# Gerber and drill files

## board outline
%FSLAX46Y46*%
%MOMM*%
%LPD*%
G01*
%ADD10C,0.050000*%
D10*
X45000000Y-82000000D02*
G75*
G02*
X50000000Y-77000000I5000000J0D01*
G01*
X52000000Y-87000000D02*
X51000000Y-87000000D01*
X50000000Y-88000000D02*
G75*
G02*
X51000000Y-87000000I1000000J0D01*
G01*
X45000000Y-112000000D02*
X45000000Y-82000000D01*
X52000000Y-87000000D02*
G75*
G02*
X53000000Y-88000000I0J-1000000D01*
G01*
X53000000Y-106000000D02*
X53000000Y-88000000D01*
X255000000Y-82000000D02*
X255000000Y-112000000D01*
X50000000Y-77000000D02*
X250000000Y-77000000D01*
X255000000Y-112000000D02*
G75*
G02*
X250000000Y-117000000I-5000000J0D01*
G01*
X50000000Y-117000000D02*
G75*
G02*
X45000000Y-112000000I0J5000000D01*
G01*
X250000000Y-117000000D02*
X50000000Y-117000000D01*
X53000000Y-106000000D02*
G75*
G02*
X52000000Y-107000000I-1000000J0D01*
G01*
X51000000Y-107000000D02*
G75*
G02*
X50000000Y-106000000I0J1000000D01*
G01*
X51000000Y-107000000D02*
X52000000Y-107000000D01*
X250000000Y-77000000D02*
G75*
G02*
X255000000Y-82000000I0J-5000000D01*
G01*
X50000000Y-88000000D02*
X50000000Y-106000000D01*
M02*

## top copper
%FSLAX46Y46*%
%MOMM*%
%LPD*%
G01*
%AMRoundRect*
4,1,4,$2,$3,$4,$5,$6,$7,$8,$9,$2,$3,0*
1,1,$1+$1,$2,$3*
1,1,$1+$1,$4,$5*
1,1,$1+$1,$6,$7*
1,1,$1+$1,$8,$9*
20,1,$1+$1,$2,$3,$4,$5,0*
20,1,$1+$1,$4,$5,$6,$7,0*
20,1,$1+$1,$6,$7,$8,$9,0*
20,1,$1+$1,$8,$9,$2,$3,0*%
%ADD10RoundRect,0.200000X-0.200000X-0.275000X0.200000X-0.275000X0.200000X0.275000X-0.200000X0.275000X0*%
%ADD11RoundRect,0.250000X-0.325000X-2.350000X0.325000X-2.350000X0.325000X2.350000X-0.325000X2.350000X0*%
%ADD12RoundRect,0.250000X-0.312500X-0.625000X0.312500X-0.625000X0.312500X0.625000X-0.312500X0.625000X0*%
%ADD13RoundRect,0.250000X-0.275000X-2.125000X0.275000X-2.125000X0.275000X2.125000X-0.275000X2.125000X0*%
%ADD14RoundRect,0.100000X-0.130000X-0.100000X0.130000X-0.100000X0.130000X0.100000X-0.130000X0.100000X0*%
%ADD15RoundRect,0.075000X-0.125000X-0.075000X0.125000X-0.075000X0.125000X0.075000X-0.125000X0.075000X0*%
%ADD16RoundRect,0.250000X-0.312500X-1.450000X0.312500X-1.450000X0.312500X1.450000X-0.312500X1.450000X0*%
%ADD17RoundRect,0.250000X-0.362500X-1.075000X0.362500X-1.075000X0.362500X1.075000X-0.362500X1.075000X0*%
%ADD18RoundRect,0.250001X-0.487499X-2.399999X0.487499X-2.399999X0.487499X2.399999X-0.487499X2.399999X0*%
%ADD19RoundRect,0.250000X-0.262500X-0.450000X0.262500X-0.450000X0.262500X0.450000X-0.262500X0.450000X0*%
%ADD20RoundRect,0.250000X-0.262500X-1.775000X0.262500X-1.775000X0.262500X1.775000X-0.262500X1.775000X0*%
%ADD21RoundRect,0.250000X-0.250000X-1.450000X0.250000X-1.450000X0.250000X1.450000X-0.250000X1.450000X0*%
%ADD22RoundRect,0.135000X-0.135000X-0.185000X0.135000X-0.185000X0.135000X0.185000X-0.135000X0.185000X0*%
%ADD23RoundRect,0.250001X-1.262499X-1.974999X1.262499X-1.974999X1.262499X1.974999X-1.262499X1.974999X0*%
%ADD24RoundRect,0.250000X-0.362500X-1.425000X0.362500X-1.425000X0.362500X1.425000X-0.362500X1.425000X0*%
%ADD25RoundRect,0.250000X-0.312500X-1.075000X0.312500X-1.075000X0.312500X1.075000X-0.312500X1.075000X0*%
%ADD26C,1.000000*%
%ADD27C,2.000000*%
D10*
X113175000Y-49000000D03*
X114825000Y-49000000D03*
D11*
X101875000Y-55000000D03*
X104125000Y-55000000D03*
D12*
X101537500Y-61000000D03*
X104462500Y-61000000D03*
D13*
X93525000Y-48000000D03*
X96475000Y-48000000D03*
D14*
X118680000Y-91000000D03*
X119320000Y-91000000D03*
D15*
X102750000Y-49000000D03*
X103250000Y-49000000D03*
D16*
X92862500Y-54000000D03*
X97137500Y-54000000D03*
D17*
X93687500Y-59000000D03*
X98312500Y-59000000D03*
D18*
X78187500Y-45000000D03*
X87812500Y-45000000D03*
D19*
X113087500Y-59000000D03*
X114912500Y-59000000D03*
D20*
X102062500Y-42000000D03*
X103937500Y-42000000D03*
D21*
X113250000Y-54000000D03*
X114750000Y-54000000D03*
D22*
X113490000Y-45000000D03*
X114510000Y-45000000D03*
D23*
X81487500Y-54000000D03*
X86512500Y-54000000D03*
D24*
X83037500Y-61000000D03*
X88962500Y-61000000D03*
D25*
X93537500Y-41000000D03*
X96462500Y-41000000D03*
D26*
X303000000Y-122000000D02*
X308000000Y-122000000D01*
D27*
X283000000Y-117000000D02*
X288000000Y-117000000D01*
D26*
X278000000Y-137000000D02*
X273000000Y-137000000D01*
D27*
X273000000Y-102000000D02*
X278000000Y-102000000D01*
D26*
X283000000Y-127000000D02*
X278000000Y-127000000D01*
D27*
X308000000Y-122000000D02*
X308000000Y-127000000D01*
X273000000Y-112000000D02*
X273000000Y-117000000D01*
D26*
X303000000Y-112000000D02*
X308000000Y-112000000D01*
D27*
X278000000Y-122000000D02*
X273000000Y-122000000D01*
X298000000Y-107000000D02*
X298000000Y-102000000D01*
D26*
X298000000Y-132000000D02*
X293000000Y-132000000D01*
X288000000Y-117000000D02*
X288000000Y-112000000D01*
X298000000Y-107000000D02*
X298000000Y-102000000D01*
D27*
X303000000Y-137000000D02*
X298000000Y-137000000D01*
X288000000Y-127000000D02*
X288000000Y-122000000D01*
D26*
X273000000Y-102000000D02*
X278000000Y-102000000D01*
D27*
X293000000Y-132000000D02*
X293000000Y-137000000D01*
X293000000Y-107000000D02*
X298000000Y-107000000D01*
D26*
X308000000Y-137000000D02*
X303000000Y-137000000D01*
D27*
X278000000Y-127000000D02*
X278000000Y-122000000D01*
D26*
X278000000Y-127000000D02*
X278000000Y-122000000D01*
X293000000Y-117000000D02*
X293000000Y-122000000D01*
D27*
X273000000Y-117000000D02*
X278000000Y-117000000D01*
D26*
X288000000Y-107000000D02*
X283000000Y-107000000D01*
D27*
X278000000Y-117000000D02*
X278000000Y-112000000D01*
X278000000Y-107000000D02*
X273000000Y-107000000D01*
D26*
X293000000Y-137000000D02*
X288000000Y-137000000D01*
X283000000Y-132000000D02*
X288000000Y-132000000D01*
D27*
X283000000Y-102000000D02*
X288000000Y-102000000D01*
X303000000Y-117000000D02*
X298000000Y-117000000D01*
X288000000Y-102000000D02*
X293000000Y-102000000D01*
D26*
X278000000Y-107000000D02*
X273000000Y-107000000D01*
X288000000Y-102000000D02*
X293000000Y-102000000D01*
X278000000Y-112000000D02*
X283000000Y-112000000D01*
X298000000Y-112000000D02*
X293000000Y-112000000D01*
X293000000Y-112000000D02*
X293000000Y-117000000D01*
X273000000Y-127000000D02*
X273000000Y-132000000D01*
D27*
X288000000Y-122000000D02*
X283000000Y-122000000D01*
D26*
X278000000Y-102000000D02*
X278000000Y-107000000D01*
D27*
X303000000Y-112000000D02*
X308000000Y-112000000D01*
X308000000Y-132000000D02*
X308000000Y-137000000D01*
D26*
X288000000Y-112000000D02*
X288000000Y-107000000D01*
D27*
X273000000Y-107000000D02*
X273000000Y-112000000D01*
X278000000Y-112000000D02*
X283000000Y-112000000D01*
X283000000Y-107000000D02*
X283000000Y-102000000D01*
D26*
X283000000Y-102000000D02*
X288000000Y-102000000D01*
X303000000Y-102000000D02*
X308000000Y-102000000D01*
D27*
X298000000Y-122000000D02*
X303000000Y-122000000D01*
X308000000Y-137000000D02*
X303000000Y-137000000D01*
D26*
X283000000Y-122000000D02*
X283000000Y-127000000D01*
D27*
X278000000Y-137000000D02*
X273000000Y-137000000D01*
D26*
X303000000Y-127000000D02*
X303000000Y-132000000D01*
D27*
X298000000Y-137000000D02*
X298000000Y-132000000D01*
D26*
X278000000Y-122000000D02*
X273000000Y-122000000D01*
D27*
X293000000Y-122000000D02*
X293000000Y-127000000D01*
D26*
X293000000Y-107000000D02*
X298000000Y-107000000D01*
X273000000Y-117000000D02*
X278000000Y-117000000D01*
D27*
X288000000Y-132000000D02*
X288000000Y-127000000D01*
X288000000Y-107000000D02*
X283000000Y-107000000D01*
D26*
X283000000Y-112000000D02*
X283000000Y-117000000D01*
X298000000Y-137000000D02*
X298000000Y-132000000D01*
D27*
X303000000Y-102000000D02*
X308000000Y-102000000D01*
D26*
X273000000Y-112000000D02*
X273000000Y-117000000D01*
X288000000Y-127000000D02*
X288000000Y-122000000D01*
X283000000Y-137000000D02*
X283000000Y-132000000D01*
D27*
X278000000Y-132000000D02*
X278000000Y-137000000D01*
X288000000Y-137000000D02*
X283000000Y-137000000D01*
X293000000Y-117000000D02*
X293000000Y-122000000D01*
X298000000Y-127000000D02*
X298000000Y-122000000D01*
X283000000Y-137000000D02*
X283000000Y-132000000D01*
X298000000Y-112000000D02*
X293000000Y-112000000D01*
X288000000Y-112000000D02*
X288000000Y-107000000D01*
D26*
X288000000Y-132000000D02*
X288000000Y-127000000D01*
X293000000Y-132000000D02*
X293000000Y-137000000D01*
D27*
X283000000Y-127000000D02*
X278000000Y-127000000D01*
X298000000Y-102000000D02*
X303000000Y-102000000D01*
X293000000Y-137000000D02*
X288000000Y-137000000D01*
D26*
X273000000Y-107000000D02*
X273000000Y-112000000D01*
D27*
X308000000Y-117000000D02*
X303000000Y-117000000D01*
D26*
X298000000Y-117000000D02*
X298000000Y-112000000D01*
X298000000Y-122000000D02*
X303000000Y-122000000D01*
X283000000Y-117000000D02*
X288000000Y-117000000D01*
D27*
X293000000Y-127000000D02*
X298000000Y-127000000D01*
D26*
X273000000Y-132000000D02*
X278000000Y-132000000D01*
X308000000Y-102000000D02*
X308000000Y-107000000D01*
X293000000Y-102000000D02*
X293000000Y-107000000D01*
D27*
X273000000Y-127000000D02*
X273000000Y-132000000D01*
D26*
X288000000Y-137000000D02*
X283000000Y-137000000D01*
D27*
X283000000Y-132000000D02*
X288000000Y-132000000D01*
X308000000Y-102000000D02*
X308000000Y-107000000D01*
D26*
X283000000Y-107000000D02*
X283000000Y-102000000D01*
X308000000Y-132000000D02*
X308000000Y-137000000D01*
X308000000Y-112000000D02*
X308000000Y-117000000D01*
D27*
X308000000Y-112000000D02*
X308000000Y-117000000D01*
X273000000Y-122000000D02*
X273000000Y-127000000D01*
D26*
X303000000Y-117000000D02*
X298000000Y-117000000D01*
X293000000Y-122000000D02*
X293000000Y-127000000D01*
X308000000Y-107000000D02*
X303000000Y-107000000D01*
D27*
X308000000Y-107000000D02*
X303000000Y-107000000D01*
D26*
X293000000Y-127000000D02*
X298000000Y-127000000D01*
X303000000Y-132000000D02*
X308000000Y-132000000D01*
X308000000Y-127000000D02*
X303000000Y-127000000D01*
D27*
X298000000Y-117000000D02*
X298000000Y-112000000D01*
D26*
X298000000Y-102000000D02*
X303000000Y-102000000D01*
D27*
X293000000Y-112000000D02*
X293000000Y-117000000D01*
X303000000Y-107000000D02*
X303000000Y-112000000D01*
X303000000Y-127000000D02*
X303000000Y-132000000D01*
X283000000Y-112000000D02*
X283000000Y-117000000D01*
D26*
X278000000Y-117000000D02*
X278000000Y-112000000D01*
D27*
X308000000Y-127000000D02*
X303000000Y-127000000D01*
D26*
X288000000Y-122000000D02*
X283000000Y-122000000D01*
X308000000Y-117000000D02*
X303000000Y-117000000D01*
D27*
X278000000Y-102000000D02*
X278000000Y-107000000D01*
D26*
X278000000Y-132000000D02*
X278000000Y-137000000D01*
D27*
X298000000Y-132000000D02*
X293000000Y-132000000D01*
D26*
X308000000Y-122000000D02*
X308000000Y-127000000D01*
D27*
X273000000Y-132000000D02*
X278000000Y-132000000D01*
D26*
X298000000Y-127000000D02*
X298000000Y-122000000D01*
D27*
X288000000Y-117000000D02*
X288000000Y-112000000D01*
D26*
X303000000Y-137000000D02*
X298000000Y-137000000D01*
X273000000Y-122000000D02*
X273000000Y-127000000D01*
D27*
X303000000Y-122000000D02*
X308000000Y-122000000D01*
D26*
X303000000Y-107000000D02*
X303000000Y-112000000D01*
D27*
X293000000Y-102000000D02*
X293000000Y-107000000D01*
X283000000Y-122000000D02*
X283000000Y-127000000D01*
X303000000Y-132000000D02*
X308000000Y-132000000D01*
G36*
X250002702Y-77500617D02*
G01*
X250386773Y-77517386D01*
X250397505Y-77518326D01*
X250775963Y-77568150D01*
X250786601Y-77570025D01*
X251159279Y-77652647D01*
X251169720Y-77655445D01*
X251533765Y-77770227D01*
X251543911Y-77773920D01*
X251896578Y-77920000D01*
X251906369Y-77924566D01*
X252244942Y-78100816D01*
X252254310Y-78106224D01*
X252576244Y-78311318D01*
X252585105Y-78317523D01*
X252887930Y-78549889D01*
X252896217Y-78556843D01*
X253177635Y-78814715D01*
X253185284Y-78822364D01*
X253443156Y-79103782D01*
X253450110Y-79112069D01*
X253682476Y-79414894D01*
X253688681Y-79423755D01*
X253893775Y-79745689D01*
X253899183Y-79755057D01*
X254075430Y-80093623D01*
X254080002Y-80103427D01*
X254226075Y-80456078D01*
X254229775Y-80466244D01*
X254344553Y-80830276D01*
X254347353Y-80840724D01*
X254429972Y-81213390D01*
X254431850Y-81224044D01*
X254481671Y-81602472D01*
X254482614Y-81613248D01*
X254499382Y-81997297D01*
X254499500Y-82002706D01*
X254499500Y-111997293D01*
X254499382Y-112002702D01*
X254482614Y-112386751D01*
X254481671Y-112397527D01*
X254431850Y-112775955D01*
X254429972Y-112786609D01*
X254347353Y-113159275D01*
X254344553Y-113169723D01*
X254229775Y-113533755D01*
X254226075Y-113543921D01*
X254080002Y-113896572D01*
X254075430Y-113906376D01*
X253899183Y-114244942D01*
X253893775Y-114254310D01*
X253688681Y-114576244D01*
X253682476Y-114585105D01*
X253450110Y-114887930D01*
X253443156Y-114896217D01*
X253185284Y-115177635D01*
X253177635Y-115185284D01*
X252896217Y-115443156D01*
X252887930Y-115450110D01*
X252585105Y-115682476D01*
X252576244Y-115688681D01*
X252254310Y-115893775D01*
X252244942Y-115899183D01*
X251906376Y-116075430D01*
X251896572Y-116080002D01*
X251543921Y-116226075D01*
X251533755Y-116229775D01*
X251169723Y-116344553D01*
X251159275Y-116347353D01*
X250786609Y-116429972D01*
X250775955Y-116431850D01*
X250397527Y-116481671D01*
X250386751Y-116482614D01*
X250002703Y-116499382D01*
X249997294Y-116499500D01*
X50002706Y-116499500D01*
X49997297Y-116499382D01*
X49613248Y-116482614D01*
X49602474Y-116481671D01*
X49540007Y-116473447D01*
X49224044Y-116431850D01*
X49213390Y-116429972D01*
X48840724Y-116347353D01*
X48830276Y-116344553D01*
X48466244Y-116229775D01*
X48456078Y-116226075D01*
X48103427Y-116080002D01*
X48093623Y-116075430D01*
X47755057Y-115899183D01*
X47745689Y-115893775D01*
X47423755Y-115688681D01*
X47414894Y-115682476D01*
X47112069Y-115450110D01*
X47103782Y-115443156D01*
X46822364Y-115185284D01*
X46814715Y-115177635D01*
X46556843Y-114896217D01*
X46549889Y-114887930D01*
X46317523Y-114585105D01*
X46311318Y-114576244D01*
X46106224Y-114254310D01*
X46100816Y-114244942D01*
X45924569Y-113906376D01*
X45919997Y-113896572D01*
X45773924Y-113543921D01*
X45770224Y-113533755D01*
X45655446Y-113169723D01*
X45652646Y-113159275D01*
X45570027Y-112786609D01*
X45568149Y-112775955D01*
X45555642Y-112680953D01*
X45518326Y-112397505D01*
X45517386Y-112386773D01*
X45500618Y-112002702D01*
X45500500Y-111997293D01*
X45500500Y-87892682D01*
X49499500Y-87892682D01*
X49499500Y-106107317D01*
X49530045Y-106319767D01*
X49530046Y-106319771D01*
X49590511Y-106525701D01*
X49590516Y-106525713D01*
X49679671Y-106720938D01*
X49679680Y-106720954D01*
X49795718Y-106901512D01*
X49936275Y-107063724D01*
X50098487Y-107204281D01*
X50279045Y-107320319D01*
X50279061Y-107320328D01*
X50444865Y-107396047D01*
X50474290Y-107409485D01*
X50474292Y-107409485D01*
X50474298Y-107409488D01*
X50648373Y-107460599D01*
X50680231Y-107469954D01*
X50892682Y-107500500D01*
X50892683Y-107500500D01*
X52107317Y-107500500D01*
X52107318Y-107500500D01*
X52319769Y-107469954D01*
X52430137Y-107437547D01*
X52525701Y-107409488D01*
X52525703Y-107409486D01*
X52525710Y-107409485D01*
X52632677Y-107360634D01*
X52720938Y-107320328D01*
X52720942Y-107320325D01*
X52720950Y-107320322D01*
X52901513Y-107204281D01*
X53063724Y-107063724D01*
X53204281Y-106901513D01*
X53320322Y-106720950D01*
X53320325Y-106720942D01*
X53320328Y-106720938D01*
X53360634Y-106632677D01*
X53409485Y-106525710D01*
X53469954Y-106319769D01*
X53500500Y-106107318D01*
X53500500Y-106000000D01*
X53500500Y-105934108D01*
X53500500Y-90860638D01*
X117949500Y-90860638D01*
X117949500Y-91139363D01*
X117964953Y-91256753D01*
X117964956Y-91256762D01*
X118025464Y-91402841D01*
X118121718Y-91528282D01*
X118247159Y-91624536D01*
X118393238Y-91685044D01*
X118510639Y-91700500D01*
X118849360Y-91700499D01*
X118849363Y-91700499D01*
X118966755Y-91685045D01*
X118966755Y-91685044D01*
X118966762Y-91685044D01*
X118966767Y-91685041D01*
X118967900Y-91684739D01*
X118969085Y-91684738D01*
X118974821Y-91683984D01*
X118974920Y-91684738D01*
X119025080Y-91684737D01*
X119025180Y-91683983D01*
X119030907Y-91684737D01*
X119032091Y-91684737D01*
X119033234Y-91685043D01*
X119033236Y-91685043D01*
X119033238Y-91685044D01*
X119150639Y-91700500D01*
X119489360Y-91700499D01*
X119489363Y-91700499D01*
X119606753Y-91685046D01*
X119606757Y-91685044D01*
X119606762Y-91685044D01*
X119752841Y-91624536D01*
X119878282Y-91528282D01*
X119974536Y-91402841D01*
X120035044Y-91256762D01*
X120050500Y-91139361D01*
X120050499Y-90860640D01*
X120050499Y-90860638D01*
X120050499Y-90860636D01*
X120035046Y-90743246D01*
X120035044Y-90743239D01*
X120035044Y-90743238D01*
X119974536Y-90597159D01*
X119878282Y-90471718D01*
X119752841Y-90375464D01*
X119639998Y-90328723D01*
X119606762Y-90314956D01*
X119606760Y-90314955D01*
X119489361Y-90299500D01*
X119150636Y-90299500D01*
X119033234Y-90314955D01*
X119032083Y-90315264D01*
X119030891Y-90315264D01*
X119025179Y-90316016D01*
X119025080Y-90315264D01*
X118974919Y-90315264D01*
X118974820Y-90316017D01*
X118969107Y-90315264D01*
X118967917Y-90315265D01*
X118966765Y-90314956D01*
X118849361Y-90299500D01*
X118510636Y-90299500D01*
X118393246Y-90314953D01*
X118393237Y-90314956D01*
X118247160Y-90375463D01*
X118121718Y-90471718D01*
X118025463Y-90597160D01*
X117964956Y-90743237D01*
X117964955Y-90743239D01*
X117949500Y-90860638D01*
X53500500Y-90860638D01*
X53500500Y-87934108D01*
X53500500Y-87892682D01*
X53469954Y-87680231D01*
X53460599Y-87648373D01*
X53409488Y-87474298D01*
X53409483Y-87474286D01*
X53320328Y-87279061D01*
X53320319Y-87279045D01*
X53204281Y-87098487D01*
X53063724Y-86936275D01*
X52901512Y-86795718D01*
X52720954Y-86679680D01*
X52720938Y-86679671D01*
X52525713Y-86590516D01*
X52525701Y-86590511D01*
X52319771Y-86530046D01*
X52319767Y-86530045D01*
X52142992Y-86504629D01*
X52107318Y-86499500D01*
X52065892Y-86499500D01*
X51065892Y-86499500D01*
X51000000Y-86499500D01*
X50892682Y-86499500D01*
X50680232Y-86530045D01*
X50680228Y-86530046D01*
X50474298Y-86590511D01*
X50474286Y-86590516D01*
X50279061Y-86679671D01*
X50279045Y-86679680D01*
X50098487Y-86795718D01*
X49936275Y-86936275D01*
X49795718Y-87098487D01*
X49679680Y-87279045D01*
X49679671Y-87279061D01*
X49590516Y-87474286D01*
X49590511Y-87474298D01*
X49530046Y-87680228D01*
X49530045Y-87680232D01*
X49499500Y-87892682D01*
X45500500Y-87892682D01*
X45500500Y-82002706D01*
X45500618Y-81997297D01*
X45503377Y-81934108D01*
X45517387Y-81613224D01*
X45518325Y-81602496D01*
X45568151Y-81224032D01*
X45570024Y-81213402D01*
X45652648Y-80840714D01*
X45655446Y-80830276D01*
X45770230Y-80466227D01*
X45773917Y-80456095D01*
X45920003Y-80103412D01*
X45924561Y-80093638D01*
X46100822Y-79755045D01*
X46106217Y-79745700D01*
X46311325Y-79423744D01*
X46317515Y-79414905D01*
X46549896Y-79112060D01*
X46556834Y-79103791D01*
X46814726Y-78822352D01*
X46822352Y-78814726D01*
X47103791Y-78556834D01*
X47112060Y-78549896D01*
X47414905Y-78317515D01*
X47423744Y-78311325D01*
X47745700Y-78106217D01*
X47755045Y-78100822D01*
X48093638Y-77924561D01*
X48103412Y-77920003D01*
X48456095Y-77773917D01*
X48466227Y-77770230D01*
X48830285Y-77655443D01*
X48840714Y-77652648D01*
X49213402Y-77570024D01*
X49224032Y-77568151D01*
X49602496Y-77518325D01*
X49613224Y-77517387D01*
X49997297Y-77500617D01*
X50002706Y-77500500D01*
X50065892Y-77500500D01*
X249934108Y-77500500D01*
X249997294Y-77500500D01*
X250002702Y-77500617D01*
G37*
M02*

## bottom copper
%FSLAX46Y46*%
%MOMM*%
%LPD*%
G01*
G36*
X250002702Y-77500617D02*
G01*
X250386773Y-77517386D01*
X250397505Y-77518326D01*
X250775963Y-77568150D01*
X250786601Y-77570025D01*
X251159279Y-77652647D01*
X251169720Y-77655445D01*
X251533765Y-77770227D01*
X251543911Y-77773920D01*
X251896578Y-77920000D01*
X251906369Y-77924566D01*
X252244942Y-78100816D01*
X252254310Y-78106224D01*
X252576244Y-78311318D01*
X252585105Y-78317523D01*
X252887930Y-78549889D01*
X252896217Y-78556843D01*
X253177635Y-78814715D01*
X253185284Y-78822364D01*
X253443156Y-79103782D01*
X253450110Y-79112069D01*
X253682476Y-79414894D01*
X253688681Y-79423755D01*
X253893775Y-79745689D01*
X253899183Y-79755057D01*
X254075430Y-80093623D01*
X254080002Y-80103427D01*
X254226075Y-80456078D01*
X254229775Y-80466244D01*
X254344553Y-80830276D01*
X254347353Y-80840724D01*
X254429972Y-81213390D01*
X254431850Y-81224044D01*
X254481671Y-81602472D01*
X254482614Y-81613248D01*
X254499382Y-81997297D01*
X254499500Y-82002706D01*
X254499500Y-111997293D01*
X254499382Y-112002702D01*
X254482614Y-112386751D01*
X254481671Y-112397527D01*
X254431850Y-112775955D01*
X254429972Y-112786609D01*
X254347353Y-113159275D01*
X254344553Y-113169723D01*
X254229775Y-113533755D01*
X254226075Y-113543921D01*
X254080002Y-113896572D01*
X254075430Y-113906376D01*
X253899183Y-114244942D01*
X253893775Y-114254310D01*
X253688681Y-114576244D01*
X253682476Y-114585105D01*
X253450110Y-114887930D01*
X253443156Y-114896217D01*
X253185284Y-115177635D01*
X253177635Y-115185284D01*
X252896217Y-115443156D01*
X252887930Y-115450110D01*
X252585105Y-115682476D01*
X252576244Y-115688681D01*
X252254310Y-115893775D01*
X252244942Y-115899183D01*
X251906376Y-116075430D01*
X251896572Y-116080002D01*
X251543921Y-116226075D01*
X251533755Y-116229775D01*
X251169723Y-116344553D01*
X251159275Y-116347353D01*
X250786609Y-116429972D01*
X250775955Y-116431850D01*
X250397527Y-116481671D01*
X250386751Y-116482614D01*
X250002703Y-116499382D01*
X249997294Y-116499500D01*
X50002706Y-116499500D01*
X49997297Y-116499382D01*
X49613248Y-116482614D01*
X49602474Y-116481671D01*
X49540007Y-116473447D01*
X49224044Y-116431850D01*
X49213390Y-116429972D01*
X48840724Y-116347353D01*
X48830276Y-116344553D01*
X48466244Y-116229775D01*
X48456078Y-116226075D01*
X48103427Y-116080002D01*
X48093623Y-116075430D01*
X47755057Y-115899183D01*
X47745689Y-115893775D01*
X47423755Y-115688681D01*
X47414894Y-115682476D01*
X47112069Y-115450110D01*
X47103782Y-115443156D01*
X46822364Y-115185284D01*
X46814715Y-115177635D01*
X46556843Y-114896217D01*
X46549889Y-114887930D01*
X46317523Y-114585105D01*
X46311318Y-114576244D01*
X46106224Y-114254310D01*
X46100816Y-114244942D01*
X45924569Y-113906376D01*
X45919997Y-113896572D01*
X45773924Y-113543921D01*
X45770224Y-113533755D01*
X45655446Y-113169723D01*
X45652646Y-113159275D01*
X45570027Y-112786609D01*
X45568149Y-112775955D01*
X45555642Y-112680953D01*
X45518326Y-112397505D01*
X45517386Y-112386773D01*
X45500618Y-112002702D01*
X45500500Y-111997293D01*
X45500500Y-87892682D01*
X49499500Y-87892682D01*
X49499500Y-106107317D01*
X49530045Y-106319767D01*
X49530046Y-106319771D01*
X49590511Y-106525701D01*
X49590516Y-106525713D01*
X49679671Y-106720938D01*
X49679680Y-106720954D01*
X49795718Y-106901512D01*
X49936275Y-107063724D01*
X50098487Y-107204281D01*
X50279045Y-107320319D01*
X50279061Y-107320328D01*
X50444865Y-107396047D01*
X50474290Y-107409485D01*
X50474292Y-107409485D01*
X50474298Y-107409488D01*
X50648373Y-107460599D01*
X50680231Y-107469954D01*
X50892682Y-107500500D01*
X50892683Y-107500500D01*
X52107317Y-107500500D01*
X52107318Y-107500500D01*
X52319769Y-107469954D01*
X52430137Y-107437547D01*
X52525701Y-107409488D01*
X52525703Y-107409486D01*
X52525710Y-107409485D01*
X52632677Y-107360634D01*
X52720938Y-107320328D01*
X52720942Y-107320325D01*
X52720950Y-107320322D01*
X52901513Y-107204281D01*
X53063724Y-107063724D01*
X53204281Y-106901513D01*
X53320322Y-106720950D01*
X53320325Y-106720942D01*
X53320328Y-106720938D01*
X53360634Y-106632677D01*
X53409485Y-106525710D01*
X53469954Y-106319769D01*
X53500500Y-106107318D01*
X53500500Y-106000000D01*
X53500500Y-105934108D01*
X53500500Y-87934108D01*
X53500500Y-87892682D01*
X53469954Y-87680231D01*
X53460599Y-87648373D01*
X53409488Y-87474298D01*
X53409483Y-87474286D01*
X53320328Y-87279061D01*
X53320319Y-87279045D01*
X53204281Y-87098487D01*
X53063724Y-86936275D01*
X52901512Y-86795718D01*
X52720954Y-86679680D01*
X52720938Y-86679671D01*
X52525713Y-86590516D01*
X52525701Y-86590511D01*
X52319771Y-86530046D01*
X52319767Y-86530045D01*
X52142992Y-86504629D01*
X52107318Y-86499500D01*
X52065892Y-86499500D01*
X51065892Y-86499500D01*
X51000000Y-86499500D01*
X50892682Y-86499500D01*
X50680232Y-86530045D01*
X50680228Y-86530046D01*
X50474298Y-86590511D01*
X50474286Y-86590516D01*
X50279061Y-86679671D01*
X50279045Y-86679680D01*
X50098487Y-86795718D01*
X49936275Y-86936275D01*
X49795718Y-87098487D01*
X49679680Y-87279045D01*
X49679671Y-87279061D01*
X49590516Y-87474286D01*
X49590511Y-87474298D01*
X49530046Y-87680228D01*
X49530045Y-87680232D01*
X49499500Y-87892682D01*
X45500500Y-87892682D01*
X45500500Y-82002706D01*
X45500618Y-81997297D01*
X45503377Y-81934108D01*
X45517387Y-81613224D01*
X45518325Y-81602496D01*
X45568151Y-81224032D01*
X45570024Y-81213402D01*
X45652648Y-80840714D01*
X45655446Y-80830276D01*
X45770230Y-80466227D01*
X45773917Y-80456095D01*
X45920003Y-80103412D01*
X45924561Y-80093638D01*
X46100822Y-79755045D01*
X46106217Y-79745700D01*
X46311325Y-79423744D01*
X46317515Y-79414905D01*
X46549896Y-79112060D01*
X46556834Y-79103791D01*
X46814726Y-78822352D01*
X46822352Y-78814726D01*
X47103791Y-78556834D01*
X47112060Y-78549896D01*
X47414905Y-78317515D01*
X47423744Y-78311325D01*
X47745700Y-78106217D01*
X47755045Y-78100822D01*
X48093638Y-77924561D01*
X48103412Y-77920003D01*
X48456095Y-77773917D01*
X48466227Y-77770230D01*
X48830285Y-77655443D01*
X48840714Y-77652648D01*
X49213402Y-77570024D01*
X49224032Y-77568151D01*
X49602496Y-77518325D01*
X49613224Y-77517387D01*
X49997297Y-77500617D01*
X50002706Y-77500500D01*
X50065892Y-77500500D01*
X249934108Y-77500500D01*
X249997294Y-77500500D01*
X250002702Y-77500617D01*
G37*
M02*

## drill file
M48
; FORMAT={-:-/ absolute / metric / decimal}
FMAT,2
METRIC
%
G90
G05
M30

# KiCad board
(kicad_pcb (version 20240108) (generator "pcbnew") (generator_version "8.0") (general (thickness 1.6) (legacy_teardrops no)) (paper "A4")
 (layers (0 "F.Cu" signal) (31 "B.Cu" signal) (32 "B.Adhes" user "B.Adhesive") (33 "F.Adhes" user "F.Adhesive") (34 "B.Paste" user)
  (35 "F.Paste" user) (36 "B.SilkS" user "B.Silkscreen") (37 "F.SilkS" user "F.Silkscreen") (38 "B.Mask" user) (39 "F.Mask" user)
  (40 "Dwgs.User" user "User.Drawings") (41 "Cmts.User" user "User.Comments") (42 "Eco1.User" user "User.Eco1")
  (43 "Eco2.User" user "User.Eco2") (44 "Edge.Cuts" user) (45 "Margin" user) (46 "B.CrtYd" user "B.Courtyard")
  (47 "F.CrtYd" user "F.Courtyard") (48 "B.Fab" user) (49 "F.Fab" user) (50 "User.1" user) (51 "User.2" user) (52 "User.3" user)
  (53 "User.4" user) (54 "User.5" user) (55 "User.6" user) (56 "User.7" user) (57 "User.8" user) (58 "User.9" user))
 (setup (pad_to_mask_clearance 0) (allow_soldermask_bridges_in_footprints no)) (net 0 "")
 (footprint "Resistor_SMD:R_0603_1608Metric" (layer "F.Cu") (at 114 49)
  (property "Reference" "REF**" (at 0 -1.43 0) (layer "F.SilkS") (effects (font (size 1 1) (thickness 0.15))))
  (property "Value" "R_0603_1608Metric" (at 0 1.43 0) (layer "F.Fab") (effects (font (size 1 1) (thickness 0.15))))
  (pad "1" smd roundrect (at -0.825 0) (size 0.8 0.95) (layers "F.Cu" "F.Paste" "F.Mask") (roundrect_rratio 0.25))
  (pad "2" smd roundrect (at 0.825 0) (size 0.8 0.95) (layers "F.Cu" "F.Paste" "F.Mask") (roundrect_rratio 0.25)))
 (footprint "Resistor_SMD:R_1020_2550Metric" (layer "F.Cu") (at 103 55)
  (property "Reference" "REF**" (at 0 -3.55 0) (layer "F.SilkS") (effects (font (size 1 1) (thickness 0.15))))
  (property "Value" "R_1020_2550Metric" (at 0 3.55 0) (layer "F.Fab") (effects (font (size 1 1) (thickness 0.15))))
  (pad "1" smd roundrect (at -1.125 0) (size 1.15 5.2) (layers "F.Cu" "F.Paste" "F.Mask") (roundrect_rratio 0.217391))
  (pad "2" smd roundrect (at 1.125 0) (size 1.15 5.2) (layers "F.Cu" "F.Paste" "F.Mask") (roundrect_rratio 0.217391)))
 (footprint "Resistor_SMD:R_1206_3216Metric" (layer "F.Cu") (at 103 61)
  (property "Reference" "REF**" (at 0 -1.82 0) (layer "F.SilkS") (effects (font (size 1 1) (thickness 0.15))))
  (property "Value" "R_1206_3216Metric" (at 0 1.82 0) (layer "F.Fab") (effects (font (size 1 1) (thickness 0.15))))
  (pad "1" smd roundrect (at -1.4625 0) (size 1.125 1.75) (layers "F.Cu" "F.Paste" "F.Mask") (roundrect_rratio 0.222222))
  (pad "2" smd roundrect (at 1.4625 0) (size 1.125 1.75) (layers "F.Cu" "F.Paste" "F.Mask") (roundrect_rratio 0.222222)))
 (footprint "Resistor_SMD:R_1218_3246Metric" (layer "F.Cu") (at 95 48)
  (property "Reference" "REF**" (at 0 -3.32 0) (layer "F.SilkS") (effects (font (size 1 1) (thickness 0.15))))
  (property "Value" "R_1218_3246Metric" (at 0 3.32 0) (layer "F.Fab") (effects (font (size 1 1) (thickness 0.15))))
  (pad "1" smd roundrect (at -1.475 0) (size 1.05 4.75) (layers "F.Cu" "F.Paste" "F.Mask") (roundrect_rratio 0.238095))
  (pad "2" smd roundrect (at 1.475 0) (size 1.05 4.75) (layers "F.Cu" "F.Paste" "F.Mask") (roundrect_rratio 0.238095)))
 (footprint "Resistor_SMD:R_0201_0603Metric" (layer "F.Cu") (at 119 91)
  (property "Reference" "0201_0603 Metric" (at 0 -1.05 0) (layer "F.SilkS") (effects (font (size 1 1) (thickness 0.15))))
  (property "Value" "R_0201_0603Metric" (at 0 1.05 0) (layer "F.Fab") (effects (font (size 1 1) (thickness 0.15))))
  (pad "" smd roundrect (at -0.345 0) (size 0.318 0.36) (layers "F.Paste") (roundrect_rratio 0.25))
  (pad "" smd roundrect (at 0.345 0) (size 0.318 0.36) (layers "F.Paste") (roundrect_rratio 0.25))
  (pad "1" smd roundrect (at -0.32 0) (size 0.46 0.4) (layers "F.Cu" "F.Mask") (roundrect_rratio 0.25))
  (pad "2" smd roundrect (at 0.32 0) (size 0.46 0.4) (layers "F.Cu" "F.Mask") (roundrect_rratio 0.25)))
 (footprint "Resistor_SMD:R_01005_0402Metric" (layer "F.Cu") (at 103 49)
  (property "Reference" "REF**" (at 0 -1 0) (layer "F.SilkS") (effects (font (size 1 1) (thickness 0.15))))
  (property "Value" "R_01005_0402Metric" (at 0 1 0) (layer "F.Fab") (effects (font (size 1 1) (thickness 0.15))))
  (pad "" smd roundrect (at -0.275 0) (size 0.27 0.27) (layers "F.Paste") (roundrect_rratio 0.25))
  (pad "" smd roundrect (at 0.275 0) (size 0.27 0.27) (layers "F.Paste") (roundrect_rratio 0.25))
  (pad "1" smd roundrect (at -0.25 0) (size 0.4 0.3) (layers "F.Cu" "F.Mask") (roundrect_rratio 0.25))
  (pad "2" smd roundrect (at 0.25 0) (size 0.4 0.3) (layers "F.Cu" "F.Mask") (roundrect_rratio 0.25)))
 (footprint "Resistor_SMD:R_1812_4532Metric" (layer "F.Cu") (at 95 54)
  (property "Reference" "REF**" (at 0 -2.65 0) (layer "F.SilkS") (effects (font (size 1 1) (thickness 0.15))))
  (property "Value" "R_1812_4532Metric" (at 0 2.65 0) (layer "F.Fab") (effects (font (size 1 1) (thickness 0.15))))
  (pad "1" smd roundrect (at -2.1375 0) (size 1.125 3.4) (layers "F.Cu" "F.Paste" "F.Mask") (roundrect_rratio 0.222222))
  (pad "2" smd roundrect (at 2.1375 0) (size 1.125 3.4) (layers "F.Cu" "F.Paste" "F.Mask") (roundrect_rratio 0.222222)))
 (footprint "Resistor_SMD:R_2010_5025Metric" (layer "F.Cu") (at 96 59)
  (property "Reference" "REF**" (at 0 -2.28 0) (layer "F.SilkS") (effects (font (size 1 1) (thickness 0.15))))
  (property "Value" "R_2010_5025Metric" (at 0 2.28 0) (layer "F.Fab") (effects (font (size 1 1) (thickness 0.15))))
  (pad "1" smd roundrect (at -2.3125 0) (size 1.225 2.65) (layers "F.Cu" "F.Paste" "F.Mask") (roundrect_rratio 0.204082))
  (pad "2" smd roundrect (at 2.3125 0) (size 1.225 2.65) (layers "F.Cu" "F.Paste" "F.Mask") (roundrect_rratio 0.204082)))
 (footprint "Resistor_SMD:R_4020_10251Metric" (layer "F.Cu") (at 83 45)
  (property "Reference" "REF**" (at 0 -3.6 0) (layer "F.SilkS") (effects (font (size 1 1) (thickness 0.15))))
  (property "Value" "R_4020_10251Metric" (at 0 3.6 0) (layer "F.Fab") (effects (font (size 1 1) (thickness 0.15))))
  (pad "1" smd roundrect (at -4.8125 0) (size 1.475 5.3) (layers "F.Cu" "F.Paste" "F.Mask") (roundrect_rratio 0.169492))
  (pad "2" smd roundrect (at 4.8125 0) (size 1.475 5.3) (layers "F.Cu" "F.Paste" "F.Mask") (roundrect_rratio 0.169492)))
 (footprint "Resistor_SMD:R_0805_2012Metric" (layer "F.Cu") (at 114 59)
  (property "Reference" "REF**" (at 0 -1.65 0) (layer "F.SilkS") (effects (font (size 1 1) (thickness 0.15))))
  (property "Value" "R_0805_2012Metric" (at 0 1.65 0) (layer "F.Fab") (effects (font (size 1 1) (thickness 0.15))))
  (pad "1" smd roundrect (at -0.9125 0) (size 1.025 1.4) (layers "F.Cu" "F.Paste" "F.Mask") (roundrect_rratio 0.243902))
  (pad "2" smd roundrect (at 0.9125 0) (size 1.025 1.4) (layers "F.Cu" "F.Paste" "F.Mask") (roundrect_rratio 0.243902)))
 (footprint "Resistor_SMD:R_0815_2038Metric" (layer "F.Cu") (at 103 42)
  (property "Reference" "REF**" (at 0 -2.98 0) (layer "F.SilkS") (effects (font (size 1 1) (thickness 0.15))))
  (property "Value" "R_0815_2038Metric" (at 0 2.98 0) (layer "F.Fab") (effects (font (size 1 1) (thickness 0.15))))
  (pad "1" smd roundrect (at -0.9375 0) (size 1.025 4.05) (layers "F.Cu" "F.Paste" "F.Mask") (roundrect_rratio 0.243902))
  (pad "2" smd roundrect (at 0.9375 0) (size 1.025 4.05) (layers "F.Cu" "F.Paste" "F.Mask") (roundrect_rratio 0.243902)))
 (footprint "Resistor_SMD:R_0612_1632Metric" (layer "F.Cu") (at 114 54)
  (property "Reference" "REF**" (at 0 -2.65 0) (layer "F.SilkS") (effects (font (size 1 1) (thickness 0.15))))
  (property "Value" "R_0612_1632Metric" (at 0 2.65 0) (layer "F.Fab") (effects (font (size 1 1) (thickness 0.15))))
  (pad "1" smd roundrect (at -0.75 0) (size 1 3.4) (layers "F.Cu" "F.Paste" "F.Mask") (roundrect_rratio 0.25))
  (pad "2" smd roundrect (at 0.75 0) (size 1 3.4) (layers "F.Cu" "F.Paste" "F.Mask") (roundrect_rratio 0.25)))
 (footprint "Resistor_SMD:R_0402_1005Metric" (layer "F.Cu") (at 114 45)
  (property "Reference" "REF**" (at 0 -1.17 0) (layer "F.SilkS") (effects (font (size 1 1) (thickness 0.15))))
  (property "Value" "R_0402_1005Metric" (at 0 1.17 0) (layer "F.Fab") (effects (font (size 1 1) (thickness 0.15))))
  (pad "1" smd roundrect (at -0.51 0) (size 0.54 0.64) (layers "F.Cu" "F.Paste" "F.Mask") (roundrect_rratio 0.25))
  (pad "2" smd roundrect (at 0.51 0) (size 0.54 0.64) (layers "F.Cu" "F.Paste" "F.Mask") (roundrect_rratio 0.25)))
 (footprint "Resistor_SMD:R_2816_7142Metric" (layer "F.Cu") (at 84 54)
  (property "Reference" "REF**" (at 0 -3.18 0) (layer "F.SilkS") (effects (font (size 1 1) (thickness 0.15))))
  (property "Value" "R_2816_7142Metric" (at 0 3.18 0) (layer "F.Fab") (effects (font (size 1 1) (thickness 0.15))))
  (pad "1" smd roundrect (at -2.5125 0) (size 3.025 4.45) (layers "F.Cu" "F.Paste" "F.Mask") (roundrect_rratio 0.082645))
  (pad "2" smd roundrect (at 2.5125 0) (size 3.025 4.45) (layers "F.Cu" "F.Paste" "F.Mask") (roundrect_rratio 0.082645)))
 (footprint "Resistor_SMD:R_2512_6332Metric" (layer "F.Cu") (at 86 61)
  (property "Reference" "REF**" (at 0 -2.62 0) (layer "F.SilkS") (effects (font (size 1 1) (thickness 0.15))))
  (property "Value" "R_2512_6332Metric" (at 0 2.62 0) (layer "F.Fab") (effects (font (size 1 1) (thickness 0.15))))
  (pad "1" smd roundrect (at -2.9625 0) (size 1.225 3.35) (layers "F.Cu" "F.Paste" "F.Mask") (roundrect_rratio 0.204082))
  (pad "2" smd roundrect (at 2.9625 0) (size 1.225 3.35) (layers "F.Cu" "F.Paste" "F.Mask") (roundrect_rratio 0.204082)))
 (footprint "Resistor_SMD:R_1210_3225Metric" (layer "F.Cu") (at 95 41)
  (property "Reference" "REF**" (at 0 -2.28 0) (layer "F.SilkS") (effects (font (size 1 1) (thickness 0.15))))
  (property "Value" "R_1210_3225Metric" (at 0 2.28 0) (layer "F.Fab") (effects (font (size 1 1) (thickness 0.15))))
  (pad "1" smd roundrect (at -1.4625 0) (size 1.125 2.65) (layers "F.Cu" "F.Paste" "F.Mask") (roundrect_rratio 0.222222))
  (pad "2" smd roundrect (at 1.4625 0) (size 1.125 2.65) (layers "F.Cu" "F.Paste" "F.Mask") (roundrect_rratio 0.222222)))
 (gr_arc (start 45 82) (mid 46.464466 78.464466) (end 50 77) (stroke (width 0.05) (type default)) (layer "Edge.Cuts"))
 (gr_line (start 52 87) (end 51 87) (stroke (width 0.05) (type default)) (layer "Edge.Cuts"))
 (gr_arc (start 50 88) (mid 50.292893 87.292893) (end 51 87) (stroke (width 0.05) (type default)) (layer "Edge.Cuts"))
 (gr_line (start 45 112) (end 45 82) (stroke (width 0.05) (type default)) (layer "Edge.Cuts"))
 (gr_arc (start 52 87) (mid 52.707107 87.292893) (end 53 88) (stroke (width 0.05) (type default)) (layer "Edge.Cuts"))
 (gr_line (start 53 106) (end 53 88) (stroke (width 0.05) (type default)) (layer "Edge.Cuts"))
 (gr_line (start 255 82) (end 255 112) (stroke (width 0.05) (type default)) (layer "Edge.Cuts"))
 (gr_line (start 50 77) (end 250 77) (stroke (width 0.05) (type default)) (layer "Edge.Cuts"))
 (gr_arc (start 255 112) (mid 253.535534 115.535534) (end 250 117) (stroke (width 0.05) (type default)) (layer "Edge.Cuts"))
 (gr_arc (start 50 117) (mid 46.464466 115.535534) (end 45 112) (stroke (width 0.05) (type default)) (layer "Edge.Cuts"))
 (gr_line (start 250 117) (end 50 117) (stroke (width 0.05) (type default)) (layer "Edge.Cuts"))
 (gr_arc (start 53 106) (mid 52.707107 106.707107) (end 52 107) (stroke (width 0.05) (type default)) (layer "Edge.Cuts"))
 (gr_arc (start 51 107) (mid 50.292893 106.707107) (end 50 106) (stroke (width 0.05) (type default)) (layer "Edge.Cuts"))
 (gr_line (start 51 107) (end 52 107) (stroke (width 0.05) (type default)) (layer "Edge.Cuts"))
 (gr_arc (start 250 77) (mid 253.535534 78.464466) (end 255 82) (stroke (width 0.05) (type default)) (layer "Edge.Cuts"))
 (gr_line (start 50 88) (end 50 106) (stroke (width 0.05) (type default)) (layer "Edge.Cuts"))
 (segment (start 303 122) (end 308 122) (width 1) (layer "F.Cu") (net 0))
 (segment (start 283 117) (end 288 117) (width 2) (layer "F.Cu") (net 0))
 (segment (start 278 137) (end 273 137) (width 1) (layer "F.Cu") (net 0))
 (segment (start 273 102) (end 278 102) (width 2) (layer "F.Cu") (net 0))
 (segment (start 283 127) (end 278 127) (width 1) (layer "F.Cu") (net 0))
 (segment (start 308 122) (end 308 127) (width 2) (layer "F.Cu") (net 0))
 (segment (start 273 112) (end 273 117) (width 2) (layer "F.Cu") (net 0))
 (segment (start 303 112) (end 308 112) (width 1) (layer "F.Cu") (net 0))
 (segment (start 278 122) (end 273 122) (width 2) (layer "F.Cu") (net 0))
 (segment (start 298 107) (end 298 102) (width 2) (layer "F.Cu") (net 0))
 (segment (start 298 132) (end 293 132) (width 1) (layer "F.Cu") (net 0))
 (segment (start 288 117) (end 288 112) (width 1) (layer "F.Cu") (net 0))
 (segment (start 298 107) (end 298 102) (width 1) (layer "F.Cu") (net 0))
 (segment (start 303 137) (end 298 137) (width 2) (layer "F.Cu") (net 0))
 (segment (start 288 127) (end 288 122) (width 2) (layer "F.Cu") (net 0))
 (segment (start 273 102) (end 278 102) (width 1) (layer "F.Cu") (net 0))
 (segment (start 293 132) (end 293 137) (width 2) (layer "F.Cu") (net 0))
 (segment (start 293 107) (end 298 107) (width 2) (layer "F.Cu") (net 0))
 (segment (start 308 137) (end 303 137) (width 1) (layer "F.Cu") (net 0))
 (segment (start 278 127) (end 278 122) (width 2) (layer "F.Cu") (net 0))
 (segment (start 278 127) (end 278 122) (width 1) (layer "F.Cu") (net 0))
 (segment (start 293 117) (end 293 122) (width 1) (layer "F.Cu") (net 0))
 (segment (start 273 117) (end 278 117) (width 2) (layer "F.Cu") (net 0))
 (segment (start 288 107) (end 283 107) (width 1) (layer "F.Cu") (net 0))
 (segment (start 278 117) (end 278 112) (width 2) (layer "F.Cu") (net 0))
 (segment (start 278 107) (end 273 107) (width 2) (layer "F.Cu") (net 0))
 (segment (start 293 137) (end 288 137) (width 1) (layer "F.Cu") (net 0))
 (segment (start 283 132) (end 288 132) (width 1) (layer "F.Cu") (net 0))
 (segment (start 283 102) (end 288 102) (width 2) (layer "F.Cu") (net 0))
 (segment (start 303 117) (end 298 117) (width 2) (layer "F.Cu") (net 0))
 (segment (start 288 102) (end 293 102) (width 2) (layer "F.Cu") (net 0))
 (segment (start 278 107) (end 273 107) (width 1) (layer "F.Cu") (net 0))
 (segment (start 288 102) (end 293 102) (width 1) (layer "F.Cu") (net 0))
 (segment (start 278 112) (end 283 112) (width 1) (layer "F.Cu") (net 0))
 (segment (start 298 112) (end 293 112) (width 1) (layer "F.Cu") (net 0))
 (segment (start 293 112) (end 293 117) (width 1) (layer "F.Cu") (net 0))
 (segment (start 273 127) (end 273 132) (width 1) (layer "F.Cu") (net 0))
 (segment (start 288 122) (end 283 122) (width 2) (layer "F.Cu") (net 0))
 (segment (start 278 102) (end 278 107) (width 1) (layer "F.Cu") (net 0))
 (segment (start 303 112) (end 308 112) (width 2) (layer "F.Cu") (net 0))
 (segment (start 308 132) (end 308 137) (width 2) (layer "F.Cu") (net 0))
 (segment (start 288 112) (end 288 107) (width 1) (layer "F.Cu") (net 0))
 (segment (start 273 107) (end 273 112) (width 2) (layer "F.Cu") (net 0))
 (segment (start 278 112) (end 283 112) (width 2) (layer "F.Cu") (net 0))
 (segment (start 283 107) (end 283 102) (width 2) (layer "F.Cu") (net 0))
 (segment (start 283 102) (end 288 102) (width 1) (layer "F.Cu") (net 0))
 (segment (start 303 102) (end 308 102) (width 1) (layer "F.Cu") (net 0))
 (segment (start 298 122) (end 303 122) (width 2) (layer "F.Cu") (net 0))
 (segment (start 308 137) (end 303 137) (width 2) (layer "F.Cu") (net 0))
 (segment (start 283 122) (end 283 127) (width 1) (layer "F.Cu") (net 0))
 (segment (start 278 137) (end 273 137) (width 2) (layer "F.Cu") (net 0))
 (segment (start 303 127) (end 303 132) (width 1) (layer "F.Cu") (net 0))
 (segment (start 298 137) (end 298 132) (width 2) (layer "F.Cu") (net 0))
 (segment (start 278 122) (end 273 122) (width 1) (layer "F.Cu") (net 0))
 (segment (start 293 122) (end 293 127) (width 2) (layer "F.Cu") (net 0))
 (segment (start 293 107) (end 298 107) (width 1) (layer "F.Cu") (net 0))
 (segment (start 273 117) (end 278 117) (width 1) (layer "F.Cu") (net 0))
 (segment (start 288 132) (end 288 127) (width 2) (layer "F.Cu") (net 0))
 (segment (start 288 107) (end 283 107) (width 2) (layer "F.Cu") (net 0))
 (segment (start 283 112) (end 283 117) (width 1) (layer "F.Cu") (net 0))
 (segment (start 298 137) (end 298 132) (width 1) (layer "F.Cu") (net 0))
 (segment (start 303 102) (end 308 102) (width 2) (layer "F.Cu") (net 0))
 (segment (start 273 112) (end 273 117) (width 1) (layer "F.Cu") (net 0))
 (segment (start 288 127) (end 288 122) (width 1) (layer "F.Cu") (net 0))
 (segment (start 283 137) (end 283 132) (width 1) (layer "F.Cu") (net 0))
 (segment (start 278 132) (end 278 137) (width 2) (layer "F.Cu") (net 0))
 (segment (start 288 137) (end 283 137) (width 2) (layer "F.Cu") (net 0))
 (segment (start 293 117) (end 293 122) (width 2) (layer "F.Cu") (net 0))
 (segment (start 298 127) (end 298 122) (width 2) (layer "F.Cu") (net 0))
 (segment (start 283 137) (end 283 132) (width 2) (layer "F.Cu") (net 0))
 (segment (start 298 112) (end 293 112) (width 2) (layer "F.Cu") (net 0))
 (segment (start 288 112) (end 288 107) (width 2) (layer "F.Cu") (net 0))
 (segment (start 288 132) (end 288 127) (width 1) (layer "F.Cu") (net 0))
 (segment (start 293 132) (end 293 137) (width 1) (layer "F.Cu") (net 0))
 (segment (start 283 127) (end 278 127) (width 2) (layer "F.Cu") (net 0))
 (segment (start 298 102) (end 303 102) (width 2) (layer "F.Cu") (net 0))
 (segment (start 293 137) (end 288 137) (width 2) (layer "F.Cu") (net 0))
 (segment (start 273 107) (end 273 112) (width 1) (layer "F.Cu") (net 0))
 (segment (start 308 117) (end 303 117) (width 2) (layer "F.Cu") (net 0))
 (segment (start 298 117) (end 298 112) (width 1) (layer "F.Cu") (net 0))
 (segment (start 298 122) (end 303 122) (width 1) (layer "F.Cu") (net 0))
 (segment (start 283 117) (end 288 117) (width 1) (layer "F.Cu") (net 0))
 (segment (start 293 127) (end 298 127) (width 2) (layer "F.Cu") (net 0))
 (segment (start 273 132) (end 278 132) (width 1) (layer "F.Cu") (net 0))
 (segment (start 308 102) (end 308 107) (width 1) (layer "F.Cu") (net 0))
 (segment (start 293 102) (end 293 107) (width 1) (layer "F.Cu") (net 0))
 (segment (start 273 127) (end 273 132) (width 2) (layer "F.Cu") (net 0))
 (segment (start 288 137) (end 283 137) (width 1) (layer "F.Cu") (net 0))
 (segment (start 283 132) (end 288 132) (width 2) (layer "F.Cu") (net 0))
 (segment (start 308 102) (end 308 107) (width 2) (layer "F.Cu") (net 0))
 (segment (start 283 107) (end 283 102) (width 1) (layer "F.Cu") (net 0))
 (segment (start 308 132) (end 308 137) (width 1) (layer "F.Cu") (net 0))
 (segment (start 308 112) (end 308 117) (width 1) (layer "F.Cu") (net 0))
 (segment (start 308 112) (end 308 117) (width 2) (layer "F.Cu") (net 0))
 (segment (start 273 122) (end 273 127) (width 2) (layer "F.Cu") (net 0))
 (segment (start 303 117) (end 298 117) (width 1) (layer "F.Cu") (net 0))
 (segment (start 293 122) (end 293 127) (width 1) (layer "F.Cu") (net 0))
 (segment (start 308 107) (end 303 107) (width 1) (layer "F.Cu") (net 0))
 (segment (start 308 107) (end 303 107) (width 2) (layer "F.Cu") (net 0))
 (segment (start 293 127) (end 298 127) (width 1) (layer "F.Cu") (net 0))
 (segment (start 303 132) (end 308 132) (width 1) (layer "F.Cu") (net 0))
 (segment (start 308 127) (end 303 127) (width 1) (layer "F.Cu") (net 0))
 (segment (start 298 117) (end 298 112) (width 2) (layer "F.Cu") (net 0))
 (segment (start 298 102) (end 303 102) (width 1) (layer "F.Cu") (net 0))
 (segment (start 293 112) (end 293 117) (width 2) (layer "F.Cu") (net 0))
 (segment (start 303 107) (end 303 112) (width 2) (layer "F.Cu") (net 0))
 (segment (start 303 127) (end 303 132) (width 2) (layer "F.Cu") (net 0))
 (segment (start 283 112) (end 283 117) (width 2) (layer "F.Cu") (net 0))
 (segment (start 278 117) (end 278 112) (width 1) (layer "F.Cu") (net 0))
 (segment (start 308 127) (end 303 127) (width 2) (layer "F.Cu") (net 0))
 (segment (start 288 122) (end 283 122) (width 1) (layer "F.Cu") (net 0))
 (segment (start 308 117) (end 303 117) (width 1) (layer "F.Cu") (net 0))
 (segment (start 278 102) (end 278 107) (width 2) (layer "F.Cu") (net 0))
 (segment (start 278 132) (end 278 137) (width 1) (layer "F.Cu") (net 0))
 (segment (start 298 132) (end 293 132) (width 2) (layer "F.Cu") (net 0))
 (segment (start 308 122) (end 308 127) (width 1) (layer "F.Cu") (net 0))
 (segment (start 273 132) (end 278 132) (width 2) (layer "F.Cu") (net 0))
 (segment (start 298 127) (end 298 122) (width 1) (layer "F.Cu") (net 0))
 (segment (start 288 117) (end 288 112) (width 2) (layer "F.Cu") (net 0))
 (segment (start 303 137) (end 298 137) (width 1) (layer "F.Cu") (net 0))
 (segment (start 273 122) (end 273 127) (width 1) (layer "F.Cu") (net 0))
 (segment (start 303 122) (end 308 122) (width 2) (layer "F.Cu") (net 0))
 (segment (start 303 107) (end 303 112) (width 1) (layer "F.Cu") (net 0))
 (segment (start 293 102) (end 293 107) (width 2) (layer "F.Cu") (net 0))
 (segment (start 283 122) (end 283 127) (width 2) (layer "F.Cu") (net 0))
 (segment (start 303 132) (end 308 132) (width 2) (layer "F.Cu") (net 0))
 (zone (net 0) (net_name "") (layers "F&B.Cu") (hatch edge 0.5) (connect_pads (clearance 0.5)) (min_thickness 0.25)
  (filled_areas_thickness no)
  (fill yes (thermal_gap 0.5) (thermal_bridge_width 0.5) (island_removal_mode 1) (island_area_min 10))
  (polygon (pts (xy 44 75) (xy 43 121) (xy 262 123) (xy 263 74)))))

